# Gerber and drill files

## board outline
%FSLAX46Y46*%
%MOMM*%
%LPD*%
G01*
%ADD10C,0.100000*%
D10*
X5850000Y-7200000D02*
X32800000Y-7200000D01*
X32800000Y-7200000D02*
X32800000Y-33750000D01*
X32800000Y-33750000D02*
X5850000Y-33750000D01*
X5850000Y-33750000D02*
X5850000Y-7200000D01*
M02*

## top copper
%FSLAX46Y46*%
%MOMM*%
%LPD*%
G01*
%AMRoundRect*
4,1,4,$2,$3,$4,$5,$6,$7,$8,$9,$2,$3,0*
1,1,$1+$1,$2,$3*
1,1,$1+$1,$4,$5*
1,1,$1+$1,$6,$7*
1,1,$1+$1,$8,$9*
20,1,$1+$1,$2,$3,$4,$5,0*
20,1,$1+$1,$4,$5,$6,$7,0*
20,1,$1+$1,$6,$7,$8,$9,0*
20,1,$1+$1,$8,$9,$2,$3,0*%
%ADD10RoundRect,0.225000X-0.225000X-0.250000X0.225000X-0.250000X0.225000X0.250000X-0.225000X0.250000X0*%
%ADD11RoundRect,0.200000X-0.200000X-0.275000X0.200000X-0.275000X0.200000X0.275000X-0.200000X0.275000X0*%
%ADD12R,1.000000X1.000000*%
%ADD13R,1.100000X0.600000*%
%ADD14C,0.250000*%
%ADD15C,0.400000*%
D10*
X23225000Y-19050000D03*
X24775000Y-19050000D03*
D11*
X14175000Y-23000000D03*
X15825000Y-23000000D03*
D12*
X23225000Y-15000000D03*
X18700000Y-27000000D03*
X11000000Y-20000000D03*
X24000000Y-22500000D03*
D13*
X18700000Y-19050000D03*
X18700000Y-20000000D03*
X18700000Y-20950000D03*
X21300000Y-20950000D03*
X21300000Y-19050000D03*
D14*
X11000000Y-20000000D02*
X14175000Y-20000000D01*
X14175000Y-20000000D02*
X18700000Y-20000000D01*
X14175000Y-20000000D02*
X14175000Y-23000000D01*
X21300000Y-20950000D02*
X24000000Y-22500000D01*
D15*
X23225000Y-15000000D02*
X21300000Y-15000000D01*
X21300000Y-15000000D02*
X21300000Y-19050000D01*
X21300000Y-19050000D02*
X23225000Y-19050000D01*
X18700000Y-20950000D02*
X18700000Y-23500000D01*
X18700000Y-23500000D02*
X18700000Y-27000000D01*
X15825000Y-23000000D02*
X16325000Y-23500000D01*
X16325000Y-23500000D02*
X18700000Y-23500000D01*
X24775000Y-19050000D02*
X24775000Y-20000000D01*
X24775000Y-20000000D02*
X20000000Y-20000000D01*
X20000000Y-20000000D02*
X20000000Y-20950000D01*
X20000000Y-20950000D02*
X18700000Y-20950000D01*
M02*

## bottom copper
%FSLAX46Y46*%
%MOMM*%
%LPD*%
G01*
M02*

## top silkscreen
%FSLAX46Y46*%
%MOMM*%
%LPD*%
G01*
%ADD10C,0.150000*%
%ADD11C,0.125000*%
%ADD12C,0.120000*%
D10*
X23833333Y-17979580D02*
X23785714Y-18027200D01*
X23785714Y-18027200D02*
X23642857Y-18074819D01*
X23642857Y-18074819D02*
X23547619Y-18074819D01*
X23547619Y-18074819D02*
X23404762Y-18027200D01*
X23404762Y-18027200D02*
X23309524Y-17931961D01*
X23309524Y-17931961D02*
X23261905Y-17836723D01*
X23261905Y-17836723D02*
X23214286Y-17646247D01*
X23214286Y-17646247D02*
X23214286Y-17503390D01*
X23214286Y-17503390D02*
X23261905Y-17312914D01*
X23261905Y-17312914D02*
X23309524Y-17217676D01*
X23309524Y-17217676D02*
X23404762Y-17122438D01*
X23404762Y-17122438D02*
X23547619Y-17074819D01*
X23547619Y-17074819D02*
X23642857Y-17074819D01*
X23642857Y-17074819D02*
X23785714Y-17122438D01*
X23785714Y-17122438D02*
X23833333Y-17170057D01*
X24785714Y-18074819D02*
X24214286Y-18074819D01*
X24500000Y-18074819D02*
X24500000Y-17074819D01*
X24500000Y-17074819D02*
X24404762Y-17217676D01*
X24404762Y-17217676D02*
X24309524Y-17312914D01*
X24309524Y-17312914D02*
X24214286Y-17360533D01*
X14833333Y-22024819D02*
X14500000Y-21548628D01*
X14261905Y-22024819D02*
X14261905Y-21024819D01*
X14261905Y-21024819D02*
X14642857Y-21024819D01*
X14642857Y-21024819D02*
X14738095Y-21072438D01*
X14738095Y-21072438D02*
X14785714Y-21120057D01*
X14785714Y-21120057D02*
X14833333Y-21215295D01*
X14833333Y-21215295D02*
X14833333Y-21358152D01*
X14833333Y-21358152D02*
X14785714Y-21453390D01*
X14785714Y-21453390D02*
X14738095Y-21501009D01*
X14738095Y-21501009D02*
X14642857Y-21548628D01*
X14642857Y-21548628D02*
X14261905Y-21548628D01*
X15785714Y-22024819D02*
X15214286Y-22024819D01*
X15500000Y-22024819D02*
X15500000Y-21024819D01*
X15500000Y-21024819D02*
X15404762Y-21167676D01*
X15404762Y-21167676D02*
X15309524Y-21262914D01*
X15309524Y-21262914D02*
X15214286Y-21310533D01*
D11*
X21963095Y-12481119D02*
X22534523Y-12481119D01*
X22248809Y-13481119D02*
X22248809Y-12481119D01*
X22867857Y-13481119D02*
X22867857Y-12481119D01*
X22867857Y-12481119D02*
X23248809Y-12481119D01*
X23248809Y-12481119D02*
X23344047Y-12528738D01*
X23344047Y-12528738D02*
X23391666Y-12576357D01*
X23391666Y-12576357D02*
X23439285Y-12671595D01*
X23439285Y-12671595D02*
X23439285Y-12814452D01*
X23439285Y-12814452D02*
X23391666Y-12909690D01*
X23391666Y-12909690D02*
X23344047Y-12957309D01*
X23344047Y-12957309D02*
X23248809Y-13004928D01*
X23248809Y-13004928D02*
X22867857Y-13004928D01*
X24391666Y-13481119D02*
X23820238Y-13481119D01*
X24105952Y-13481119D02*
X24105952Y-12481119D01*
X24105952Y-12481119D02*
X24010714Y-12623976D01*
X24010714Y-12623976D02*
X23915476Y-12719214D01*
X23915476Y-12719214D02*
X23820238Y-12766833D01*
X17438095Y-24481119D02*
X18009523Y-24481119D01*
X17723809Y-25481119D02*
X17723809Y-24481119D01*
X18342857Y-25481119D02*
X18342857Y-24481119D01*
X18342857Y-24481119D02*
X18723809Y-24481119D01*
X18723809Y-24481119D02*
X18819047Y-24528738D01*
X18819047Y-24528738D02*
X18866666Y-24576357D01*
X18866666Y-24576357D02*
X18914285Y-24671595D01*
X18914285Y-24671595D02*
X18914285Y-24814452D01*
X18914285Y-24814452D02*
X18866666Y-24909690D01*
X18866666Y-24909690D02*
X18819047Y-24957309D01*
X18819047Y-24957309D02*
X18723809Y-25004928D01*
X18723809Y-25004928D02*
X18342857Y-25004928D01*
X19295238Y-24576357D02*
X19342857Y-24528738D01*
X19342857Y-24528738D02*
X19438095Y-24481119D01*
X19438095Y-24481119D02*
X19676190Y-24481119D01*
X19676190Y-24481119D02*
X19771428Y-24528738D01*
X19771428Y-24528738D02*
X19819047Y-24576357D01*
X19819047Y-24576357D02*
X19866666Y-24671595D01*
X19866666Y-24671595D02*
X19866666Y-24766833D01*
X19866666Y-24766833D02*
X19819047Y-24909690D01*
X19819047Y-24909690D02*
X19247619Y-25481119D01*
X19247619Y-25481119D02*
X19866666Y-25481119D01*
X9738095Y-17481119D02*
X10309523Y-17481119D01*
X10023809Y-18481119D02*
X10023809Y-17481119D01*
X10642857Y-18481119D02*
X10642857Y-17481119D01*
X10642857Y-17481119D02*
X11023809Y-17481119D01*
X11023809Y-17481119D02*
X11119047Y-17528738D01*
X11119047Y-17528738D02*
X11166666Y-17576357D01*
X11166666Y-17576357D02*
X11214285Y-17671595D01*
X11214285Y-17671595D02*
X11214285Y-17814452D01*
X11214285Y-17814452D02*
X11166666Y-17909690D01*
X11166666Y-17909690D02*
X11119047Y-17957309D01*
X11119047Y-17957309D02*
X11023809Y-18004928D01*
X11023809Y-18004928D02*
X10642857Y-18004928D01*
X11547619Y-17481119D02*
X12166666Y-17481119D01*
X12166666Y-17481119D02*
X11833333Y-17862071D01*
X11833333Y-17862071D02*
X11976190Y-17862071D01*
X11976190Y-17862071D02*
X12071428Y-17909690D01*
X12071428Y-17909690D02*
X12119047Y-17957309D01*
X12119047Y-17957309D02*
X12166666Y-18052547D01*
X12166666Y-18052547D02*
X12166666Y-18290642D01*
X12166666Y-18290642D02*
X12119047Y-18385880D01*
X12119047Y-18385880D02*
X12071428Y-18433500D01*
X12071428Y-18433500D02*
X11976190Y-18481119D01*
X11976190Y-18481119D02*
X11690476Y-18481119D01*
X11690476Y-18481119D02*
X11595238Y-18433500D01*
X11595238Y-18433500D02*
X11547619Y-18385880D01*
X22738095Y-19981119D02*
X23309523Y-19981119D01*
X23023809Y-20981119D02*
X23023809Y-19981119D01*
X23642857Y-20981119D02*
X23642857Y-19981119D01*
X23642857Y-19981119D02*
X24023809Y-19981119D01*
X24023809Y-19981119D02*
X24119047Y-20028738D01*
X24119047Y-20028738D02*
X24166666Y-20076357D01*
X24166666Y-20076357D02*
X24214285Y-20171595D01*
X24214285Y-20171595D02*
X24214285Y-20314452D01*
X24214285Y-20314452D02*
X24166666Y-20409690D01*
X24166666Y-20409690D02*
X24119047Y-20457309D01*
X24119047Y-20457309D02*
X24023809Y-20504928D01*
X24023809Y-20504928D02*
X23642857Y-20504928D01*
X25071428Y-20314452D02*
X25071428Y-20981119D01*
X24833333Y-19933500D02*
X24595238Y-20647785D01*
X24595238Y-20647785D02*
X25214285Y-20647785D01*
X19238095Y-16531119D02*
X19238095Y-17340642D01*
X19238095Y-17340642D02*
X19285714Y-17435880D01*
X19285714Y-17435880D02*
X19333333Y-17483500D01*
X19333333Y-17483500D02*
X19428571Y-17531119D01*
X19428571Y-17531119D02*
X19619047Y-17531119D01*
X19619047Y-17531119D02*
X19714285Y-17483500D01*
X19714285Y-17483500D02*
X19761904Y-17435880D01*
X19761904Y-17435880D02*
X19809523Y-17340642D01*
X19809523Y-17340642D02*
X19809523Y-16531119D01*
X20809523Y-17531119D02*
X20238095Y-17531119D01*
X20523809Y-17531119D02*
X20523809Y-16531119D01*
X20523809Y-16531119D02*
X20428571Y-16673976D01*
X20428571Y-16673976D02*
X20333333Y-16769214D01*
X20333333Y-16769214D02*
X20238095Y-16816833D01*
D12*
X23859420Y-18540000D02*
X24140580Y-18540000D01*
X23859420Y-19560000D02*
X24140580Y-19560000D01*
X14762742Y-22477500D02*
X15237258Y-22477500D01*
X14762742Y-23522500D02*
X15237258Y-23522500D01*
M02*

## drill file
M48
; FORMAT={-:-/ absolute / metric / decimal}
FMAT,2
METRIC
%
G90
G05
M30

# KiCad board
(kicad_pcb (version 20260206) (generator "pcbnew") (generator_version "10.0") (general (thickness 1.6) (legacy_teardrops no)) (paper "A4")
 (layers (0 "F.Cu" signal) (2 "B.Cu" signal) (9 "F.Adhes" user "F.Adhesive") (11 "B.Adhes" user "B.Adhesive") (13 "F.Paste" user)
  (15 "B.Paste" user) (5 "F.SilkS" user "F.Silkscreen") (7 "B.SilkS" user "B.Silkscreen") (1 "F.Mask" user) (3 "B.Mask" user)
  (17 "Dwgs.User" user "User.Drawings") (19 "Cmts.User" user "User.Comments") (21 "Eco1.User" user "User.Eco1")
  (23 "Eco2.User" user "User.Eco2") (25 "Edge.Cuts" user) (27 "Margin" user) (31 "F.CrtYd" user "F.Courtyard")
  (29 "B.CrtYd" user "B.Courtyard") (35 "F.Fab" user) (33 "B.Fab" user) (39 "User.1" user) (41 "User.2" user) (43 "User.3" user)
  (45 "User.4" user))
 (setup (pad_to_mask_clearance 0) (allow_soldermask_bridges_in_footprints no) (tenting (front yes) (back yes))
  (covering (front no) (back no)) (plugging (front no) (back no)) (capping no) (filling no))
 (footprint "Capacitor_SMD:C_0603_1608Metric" (layer "F.Cu") (at 24 19.05)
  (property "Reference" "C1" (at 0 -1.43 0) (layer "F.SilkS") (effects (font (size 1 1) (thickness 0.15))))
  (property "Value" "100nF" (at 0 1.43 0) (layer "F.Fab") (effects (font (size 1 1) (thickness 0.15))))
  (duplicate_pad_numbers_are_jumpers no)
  (fp_line (start -0.14058 -0.51) (end 0.14058 -0.51) (stroke (width 0.12) (type solid)) (layer "F.SilkS"))
  (fp_line (start -0.14058 0.51) (end 0.14058 0.51) (stroke (width 0.12) (type solid)) (layer "F.SilkS"))
  (pad "1" smd roundrect (at -0.775 0) (size 0.9 0.95) (layers "F.Cu" "F.Mask" "F.Paste") (roundrect_rratio 0.25) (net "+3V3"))
  (pad "2" smd roundrect (at 0.775 0) (size 0.9 0.95) (layers "F.Cu" "F.Mask" "F.Paste") (roundrect_rratio 0.25) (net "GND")))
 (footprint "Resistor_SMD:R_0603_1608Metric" (layer "F.Cu") (at 15 23)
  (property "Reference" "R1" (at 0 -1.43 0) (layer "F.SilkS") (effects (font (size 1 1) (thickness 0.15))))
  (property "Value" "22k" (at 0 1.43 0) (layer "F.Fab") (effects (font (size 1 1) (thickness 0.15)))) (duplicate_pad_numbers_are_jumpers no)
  (fp_line (start -0.237258 -0.5225) (end 0.237258 -0.5225) (stroke (width 0.12) (type solid)) (layer "F.SilkS"))
  (fp_line (start -0.237258 0.5225) (end 0.237258 0.5225) (stroke (width 0.12) (type solid)) (layer "F.SilkS"))
  (pad "1" smd roundrect (at -0.825 0) (size 0.8 0.95) (layers "F.Cu" "F.Mask" "F.Paste") (roundrect_rratio 0.25) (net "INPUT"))
  (pad "2" smd roundrect (at 0.825 0) (size 0.8 0.95) (layers "F.Cu" "F.Mask" "F.Paste") (roundrect_rratio 0.25) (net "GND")))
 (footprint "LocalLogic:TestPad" (layer "F.Cu") (at 23.225 15)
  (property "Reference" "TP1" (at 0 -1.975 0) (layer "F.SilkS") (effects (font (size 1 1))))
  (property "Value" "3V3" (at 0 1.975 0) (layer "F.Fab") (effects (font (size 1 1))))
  (pad "1" smd rect (at 0 0) (size 1 1) (layers "F.Cu" "F.Paste" "F.Mask") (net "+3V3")))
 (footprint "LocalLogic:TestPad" (layer "F.Cu") (at 18.7 27)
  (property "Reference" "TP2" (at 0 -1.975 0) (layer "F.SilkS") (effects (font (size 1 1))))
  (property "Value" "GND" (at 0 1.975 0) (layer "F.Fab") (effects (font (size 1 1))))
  (pad "1" smd rect (at 0 0) (size 1 1) (layers "F.Cu" "F.Paste" "F.Mask") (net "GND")))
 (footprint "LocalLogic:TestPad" (layer "F.Cu") (at 11 20)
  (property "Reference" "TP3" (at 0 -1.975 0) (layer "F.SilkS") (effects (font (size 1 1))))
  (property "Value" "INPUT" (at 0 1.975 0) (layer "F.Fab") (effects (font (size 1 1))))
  (pad "1" smd rect (at 0 0) (size 1 1) (layers "F.Cu" "F.Paste" "F.Mask") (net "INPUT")))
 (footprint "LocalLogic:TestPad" (layer "F.Cu") (at 24 22.5)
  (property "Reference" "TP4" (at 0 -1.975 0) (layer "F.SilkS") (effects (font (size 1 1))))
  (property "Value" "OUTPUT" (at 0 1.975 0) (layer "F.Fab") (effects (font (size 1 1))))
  (pad "1" smd rect (at 0 0) (size 1 1) (layers "F.Cu" "F.Paste" "F.Mask") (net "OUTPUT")))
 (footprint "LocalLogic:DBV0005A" (layer "F.Cu") (at 20 20)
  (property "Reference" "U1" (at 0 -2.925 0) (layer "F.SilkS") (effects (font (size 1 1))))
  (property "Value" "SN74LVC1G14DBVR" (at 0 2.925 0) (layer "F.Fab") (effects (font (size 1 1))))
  (pad "1" smd rect (at -1.3 -0.95) (size 1.1 0.6) (layers "F.Cu" "F.Paste" "F.Mask") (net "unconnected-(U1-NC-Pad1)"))
  (pad "2" smd rect (at -1.3 0) (size 1.1 0.6) (layers "F.Cu" "F.Paste" "F.Mask") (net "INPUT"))
  (pad "3" smd rect (at -1.3 0.95) (size 1.1 0.6) (layers "F.Cu" "F.Paste" "F.Mask") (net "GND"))
  (pad "4" smd rect (at 1.3 0.95) (size 1.1 0.6) (layers "F.Cu" "F.Paste" "F.Mask") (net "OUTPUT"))
  (pad "5" smd rect (at 1.3 -0.95) (size 1.1 0.6) (layers "F.Cu" "F.Paste" "F.Mask") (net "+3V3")))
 (gr_line (start 5.85 7.2) (end 32.8 7.2) (stroke (width 0.1) (type default)) (layer "Edge.Cuts"))
 (gr_line (start 32.8 7.2) (end 32.8 33.75) (stroke (width 0.1) (type default)) (layer "Edge.Cuts"))
 (gr_line (start 32.8 33.75) (end 5.85 33.75) (stroke (width 0.1) (type default)) (layer "Edge.Cuts"))
 (gr_line (start 5.85 33.75) (end 5.85 7.2) (stroke (width 0.1) (type default)) (layer "Edge.Cuts"))
 (segment (start 11.000000 20.000000) (end 14.175000 20.000000) (width 0.250000) (layer "F.Cu") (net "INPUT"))
 (segment (start 14.175000 20.000000) (end 18.700000 20.000000) (width 0.250000) (layer "F.Cu") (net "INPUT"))
 (segment (start 14.175000 20.000000) (end 14.175000 23.000000) (width 0.250000) (layer "F.Cu") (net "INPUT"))
 (segment (start 21.300000 20.950000) (end 24.000000 22.500000) (width 0.250000) (layer "F.Cu") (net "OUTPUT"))
 (segment (start 23.225000 15.000000) (end 21.300000 15.000000) (width 0.400000) (layer "F.Cu") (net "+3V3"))
 (segment (start 21.300000 15.000000) (end 21.300000 19.050000) (width 0.400000) (layer "F.Cu") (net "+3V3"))
 (segment (start 21.300000 19.050000) (end 23.225000 19.050000) (width 0.400000) (layer "F.Cu") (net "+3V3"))
 (segment (start 18.700000 20.950000) (end 18.700000 23.500000) (width 0.400000) (layer "F.Cu") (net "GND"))
 (segment (start 18.700000 23.500000) (end 18.700000 27.000000) (width 0.400000) (layer "F.Cu") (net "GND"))
 (segment (start 15.825000 23.000000) (end 16.325000 23.500000) (width 0.400000) (layer "F.Cu") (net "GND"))
 (segment (start 16.325000 23.500000) (end 18.700000 23.500000) (width 0.400000) (layer "F.Cu") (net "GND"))
 (segment (start 24.775000 19.050000) (end 24.775000 20.000000) (width 0.400000) (layer "F.Cu") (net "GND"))
 (segment (start 24.775000 20.000000) (end 20.000000 20.000000) (width 0.400000) (layer "F.Cu") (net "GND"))
 (segment (start 20.000000 20.000000) (end 20.000000 20.950000) (width 0.400000) (layer "F.Cu") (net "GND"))
 (segment (start 20.000000 20.950000) (end 18.700000 20.950000) (width 0.400000) (layer "F.Cu") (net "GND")))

